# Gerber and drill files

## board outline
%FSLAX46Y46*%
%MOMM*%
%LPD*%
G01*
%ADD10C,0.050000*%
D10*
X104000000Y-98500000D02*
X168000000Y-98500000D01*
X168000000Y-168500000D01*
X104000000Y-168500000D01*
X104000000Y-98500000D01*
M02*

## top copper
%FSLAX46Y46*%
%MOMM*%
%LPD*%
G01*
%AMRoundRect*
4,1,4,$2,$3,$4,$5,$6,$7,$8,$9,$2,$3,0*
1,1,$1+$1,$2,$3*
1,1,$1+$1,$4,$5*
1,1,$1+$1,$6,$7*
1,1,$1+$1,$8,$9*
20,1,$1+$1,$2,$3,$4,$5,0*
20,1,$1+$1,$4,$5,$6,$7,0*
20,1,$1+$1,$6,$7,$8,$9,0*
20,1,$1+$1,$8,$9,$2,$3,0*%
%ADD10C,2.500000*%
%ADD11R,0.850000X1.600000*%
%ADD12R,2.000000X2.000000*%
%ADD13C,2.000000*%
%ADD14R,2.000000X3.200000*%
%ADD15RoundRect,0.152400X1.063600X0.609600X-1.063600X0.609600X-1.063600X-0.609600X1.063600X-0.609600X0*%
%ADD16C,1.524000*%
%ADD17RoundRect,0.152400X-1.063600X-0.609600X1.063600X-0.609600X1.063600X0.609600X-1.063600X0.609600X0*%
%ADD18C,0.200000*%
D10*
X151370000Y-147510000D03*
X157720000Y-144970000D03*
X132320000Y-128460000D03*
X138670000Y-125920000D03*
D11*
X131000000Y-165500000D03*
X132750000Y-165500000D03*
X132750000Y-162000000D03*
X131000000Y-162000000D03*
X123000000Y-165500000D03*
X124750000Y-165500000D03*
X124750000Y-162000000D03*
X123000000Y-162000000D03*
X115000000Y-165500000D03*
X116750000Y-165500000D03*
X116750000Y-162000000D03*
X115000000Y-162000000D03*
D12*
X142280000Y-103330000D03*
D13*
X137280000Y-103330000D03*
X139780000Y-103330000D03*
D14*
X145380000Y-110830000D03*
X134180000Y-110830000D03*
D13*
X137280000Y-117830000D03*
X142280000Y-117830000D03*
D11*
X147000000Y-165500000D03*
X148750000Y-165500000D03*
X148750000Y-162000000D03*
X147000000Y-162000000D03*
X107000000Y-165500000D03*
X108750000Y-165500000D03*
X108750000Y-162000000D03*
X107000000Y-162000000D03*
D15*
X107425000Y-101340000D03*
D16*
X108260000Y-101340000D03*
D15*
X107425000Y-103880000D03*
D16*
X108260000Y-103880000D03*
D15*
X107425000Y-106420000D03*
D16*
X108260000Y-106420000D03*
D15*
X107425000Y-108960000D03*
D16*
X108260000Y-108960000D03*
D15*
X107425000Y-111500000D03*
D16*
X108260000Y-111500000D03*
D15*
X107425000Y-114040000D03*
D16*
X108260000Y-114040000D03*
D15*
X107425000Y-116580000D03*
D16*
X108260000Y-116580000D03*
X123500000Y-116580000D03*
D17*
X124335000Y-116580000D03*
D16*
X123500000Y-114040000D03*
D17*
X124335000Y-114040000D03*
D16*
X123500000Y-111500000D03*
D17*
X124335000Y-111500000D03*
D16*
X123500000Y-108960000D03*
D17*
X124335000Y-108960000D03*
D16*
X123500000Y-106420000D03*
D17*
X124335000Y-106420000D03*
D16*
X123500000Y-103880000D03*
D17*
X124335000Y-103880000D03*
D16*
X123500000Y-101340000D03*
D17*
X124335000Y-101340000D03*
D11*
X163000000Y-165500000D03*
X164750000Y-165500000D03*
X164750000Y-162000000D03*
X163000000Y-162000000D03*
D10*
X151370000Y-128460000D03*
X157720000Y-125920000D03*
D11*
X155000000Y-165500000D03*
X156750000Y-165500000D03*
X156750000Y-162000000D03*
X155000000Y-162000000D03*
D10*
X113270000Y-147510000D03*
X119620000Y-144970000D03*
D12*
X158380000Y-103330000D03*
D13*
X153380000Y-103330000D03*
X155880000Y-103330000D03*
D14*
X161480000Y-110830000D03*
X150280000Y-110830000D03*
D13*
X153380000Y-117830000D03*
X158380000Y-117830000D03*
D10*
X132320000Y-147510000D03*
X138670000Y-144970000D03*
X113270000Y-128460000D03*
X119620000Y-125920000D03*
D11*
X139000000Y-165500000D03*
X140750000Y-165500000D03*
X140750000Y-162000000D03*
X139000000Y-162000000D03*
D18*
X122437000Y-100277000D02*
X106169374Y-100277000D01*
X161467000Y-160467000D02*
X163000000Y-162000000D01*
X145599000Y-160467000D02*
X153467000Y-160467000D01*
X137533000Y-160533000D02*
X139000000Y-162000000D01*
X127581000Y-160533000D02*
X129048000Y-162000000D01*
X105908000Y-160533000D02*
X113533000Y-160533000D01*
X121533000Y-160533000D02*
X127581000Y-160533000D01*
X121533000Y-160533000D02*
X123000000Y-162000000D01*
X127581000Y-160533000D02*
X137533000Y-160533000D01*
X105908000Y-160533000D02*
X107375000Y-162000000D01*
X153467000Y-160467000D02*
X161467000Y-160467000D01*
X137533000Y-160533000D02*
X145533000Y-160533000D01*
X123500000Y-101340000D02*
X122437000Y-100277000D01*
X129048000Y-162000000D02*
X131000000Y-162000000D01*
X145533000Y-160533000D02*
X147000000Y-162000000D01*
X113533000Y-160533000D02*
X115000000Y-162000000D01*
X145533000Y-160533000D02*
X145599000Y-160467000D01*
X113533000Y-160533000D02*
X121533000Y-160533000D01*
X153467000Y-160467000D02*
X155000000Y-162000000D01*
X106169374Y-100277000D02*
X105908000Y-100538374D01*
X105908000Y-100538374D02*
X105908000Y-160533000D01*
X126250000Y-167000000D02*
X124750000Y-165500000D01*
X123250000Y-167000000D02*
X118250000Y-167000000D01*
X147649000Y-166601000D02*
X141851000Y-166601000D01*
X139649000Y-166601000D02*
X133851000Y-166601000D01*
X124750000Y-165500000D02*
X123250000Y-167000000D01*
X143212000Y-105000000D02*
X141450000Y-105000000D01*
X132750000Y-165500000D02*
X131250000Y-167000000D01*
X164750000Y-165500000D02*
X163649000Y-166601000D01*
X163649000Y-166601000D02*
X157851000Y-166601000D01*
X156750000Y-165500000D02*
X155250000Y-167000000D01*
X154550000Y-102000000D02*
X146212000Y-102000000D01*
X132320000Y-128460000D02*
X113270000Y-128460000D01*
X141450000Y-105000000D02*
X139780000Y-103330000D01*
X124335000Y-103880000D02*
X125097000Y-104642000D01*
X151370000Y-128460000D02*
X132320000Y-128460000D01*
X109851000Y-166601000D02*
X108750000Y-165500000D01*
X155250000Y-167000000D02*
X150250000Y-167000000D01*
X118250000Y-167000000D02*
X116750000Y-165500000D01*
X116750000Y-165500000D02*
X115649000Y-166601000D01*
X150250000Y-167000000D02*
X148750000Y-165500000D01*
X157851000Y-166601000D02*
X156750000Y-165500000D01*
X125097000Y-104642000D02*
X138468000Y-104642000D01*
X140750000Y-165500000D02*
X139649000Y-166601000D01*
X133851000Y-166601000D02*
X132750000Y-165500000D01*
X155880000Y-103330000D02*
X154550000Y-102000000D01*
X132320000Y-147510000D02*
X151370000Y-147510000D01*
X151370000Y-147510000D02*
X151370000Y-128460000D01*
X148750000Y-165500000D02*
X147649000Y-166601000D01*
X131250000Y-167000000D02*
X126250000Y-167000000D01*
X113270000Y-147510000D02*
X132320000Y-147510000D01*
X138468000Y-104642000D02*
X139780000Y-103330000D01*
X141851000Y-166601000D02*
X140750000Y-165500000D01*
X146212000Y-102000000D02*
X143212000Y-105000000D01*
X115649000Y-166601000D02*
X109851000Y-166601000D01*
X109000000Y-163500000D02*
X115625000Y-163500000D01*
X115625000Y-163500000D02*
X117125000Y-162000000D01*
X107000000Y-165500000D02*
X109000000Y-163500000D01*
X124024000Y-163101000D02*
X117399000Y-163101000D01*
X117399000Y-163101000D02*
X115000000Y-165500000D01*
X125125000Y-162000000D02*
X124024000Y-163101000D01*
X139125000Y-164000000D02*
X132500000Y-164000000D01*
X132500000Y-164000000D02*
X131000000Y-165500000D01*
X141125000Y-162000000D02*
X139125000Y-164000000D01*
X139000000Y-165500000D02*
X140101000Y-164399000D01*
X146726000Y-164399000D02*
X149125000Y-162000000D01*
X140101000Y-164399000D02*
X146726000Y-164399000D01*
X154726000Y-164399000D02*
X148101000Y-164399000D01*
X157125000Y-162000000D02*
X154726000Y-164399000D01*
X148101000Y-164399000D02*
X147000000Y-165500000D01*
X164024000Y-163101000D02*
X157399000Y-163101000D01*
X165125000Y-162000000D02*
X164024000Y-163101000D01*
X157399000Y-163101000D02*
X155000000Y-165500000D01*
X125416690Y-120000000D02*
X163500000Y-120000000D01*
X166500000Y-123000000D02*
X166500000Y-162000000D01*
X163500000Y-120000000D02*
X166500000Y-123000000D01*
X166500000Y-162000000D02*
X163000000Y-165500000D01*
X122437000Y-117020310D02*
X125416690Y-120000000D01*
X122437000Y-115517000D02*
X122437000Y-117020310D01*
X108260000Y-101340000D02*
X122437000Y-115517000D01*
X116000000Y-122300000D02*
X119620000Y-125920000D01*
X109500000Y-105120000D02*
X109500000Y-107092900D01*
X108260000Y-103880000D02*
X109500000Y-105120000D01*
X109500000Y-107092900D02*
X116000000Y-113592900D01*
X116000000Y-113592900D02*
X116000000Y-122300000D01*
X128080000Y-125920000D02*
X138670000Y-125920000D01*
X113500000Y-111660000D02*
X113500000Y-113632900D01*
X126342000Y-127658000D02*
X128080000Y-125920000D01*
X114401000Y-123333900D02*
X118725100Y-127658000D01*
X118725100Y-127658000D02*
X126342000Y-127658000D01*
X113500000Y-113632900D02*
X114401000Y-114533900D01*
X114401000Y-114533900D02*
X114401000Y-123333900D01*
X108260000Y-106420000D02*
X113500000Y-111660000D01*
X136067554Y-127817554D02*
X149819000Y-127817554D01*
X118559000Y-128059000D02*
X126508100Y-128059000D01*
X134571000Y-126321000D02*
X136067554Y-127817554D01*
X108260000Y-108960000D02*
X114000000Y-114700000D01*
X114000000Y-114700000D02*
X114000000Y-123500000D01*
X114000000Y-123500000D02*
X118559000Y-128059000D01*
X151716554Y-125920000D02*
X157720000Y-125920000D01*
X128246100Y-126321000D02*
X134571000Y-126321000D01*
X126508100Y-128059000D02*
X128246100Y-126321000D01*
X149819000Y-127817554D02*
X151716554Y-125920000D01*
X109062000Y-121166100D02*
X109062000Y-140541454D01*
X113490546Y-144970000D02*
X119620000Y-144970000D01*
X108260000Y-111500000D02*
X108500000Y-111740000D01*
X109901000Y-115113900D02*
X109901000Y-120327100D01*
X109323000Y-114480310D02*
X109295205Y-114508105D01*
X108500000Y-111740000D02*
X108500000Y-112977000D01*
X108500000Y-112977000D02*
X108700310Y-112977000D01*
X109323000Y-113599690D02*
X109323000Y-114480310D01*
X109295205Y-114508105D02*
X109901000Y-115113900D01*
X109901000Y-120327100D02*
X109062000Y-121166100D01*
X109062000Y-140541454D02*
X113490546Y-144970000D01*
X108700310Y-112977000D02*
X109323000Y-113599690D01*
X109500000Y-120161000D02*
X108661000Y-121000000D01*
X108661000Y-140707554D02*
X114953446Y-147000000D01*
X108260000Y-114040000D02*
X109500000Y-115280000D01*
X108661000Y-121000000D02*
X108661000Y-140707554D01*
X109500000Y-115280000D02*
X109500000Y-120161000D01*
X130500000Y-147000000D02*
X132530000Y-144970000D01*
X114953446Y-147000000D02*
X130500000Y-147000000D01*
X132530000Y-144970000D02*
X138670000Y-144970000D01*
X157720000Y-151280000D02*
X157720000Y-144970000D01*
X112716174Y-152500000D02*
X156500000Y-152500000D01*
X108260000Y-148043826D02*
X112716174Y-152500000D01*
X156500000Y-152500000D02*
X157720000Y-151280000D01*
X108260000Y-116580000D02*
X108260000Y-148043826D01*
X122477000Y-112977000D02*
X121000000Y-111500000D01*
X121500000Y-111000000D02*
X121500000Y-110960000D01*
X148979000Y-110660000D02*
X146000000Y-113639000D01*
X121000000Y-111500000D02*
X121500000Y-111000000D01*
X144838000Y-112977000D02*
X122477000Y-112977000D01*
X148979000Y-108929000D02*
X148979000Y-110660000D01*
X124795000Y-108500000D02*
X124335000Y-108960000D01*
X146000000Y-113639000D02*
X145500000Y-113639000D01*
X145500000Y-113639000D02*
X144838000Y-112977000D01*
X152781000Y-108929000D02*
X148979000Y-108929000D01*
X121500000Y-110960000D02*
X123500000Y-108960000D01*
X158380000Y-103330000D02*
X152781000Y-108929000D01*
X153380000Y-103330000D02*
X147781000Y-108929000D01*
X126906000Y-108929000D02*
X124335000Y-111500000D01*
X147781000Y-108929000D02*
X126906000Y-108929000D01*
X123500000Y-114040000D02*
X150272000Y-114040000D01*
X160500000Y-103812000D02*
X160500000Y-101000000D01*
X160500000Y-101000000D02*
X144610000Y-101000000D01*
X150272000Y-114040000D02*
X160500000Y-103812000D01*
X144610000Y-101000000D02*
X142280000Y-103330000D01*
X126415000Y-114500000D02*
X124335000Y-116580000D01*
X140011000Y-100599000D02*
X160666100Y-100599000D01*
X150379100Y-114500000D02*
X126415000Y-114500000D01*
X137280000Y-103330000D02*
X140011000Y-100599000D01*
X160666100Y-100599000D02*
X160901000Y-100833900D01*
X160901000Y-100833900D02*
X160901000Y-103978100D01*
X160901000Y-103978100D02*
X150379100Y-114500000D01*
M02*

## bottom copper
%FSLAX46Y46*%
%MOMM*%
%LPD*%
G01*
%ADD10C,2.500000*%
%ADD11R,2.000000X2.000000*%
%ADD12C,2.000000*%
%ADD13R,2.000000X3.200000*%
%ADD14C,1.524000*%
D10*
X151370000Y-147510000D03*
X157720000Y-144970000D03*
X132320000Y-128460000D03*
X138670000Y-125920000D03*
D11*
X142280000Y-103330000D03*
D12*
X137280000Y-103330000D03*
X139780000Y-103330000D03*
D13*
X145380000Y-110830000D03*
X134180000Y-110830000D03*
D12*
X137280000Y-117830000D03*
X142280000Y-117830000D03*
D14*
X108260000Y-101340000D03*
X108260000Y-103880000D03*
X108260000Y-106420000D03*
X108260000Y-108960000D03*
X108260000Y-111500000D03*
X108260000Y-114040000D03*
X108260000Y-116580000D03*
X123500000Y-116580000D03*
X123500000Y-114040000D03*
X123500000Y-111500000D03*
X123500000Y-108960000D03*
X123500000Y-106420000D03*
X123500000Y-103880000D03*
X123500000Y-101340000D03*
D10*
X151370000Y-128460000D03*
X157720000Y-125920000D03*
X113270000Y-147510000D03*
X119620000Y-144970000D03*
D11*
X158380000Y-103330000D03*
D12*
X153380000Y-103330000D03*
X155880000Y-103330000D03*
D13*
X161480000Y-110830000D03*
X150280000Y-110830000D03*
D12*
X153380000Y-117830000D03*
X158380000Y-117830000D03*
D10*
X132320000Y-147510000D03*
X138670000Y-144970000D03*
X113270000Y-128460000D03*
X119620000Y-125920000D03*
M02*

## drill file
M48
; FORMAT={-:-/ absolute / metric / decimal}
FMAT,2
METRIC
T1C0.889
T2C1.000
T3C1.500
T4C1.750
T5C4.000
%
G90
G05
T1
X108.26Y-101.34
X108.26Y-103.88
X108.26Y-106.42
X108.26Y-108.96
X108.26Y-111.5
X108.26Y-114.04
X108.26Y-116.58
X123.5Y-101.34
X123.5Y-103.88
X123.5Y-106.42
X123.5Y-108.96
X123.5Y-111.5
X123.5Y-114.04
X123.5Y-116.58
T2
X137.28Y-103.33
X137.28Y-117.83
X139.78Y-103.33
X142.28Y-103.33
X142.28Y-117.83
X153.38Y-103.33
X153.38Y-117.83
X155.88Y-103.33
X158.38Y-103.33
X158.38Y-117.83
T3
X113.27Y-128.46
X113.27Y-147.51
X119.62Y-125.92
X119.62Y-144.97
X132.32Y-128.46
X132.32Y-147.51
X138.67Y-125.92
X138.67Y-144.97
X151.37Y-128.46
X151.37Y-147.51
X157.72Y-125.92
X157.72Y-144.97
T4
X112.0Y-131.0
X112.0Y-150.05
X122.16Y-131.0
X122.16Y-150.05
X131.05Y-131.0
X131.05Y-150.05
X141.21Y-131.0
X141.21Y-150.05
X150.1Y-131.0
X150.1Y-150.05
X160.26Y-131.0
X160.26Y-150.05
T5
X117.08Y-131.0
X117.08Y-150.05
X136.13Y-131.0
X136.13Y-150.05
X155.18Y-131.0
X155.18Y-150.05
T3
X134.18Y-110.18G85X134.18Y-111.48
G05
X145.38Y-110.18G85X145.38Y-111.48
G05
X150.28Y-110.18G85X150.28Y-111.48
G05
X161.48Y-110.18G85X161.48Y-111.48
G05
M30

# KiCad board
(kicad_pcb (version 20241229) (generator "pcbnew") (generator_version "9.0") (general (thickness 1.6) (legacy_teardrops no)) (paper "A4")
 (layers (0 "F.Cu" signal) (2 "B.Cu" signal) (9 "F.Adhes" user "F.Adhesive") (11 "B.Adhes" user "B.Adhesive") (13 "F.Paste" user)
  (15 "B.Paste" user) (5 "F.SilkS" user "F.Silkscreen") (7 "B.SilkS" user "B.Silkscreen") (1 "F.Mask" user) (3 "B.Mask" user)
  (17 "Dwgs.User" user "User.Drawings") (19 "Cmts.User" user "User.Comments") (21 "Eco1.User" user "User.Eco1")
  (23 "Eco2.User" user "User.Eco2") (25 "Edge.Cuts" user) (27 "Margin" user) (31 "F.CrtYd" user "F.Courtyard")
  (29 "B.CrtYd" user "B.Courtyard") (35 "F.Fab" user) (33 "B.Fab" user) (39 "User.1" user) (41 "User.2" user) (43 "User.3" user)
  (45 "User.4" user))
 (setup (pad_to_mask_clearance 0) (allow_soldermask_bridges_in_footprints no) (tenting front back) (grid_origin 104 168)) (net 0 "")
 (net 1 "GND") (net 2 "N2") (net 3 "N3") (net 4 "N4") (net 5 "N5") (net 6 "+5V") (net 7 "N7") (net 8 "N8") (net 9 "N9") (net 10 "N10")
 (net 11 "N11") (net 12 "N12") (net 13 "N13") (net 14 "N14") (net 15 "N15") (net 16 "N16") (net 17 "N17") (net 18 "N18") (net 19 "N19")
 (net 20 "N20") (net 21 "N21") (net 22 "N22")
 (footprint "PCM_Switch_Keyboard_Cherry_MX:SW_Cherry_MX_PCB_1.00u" (layer "F.Cu") (at 155.18 150.05)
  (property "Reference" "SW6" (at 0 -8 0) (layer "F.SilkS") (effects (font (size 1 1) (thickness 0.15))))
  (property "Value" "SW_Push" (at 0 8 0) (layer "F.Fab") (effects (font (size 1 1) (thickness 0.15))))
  (pad "" np_thru_hole circle (at -5.08 0) (size 1.75 1.75) (drill 1.75) (layers "*.Cu" "*.Mask"))
  (pad "" np_thru_hole circle (at 0 0) (size 4 4) (drill 4) (layers "*.Cu" "*.Mask"))
  (pad "" np_thru_hole circle (at 5.08 0) (size 1.75 1.75) (drill 1.75) (layers "*.Cu" "*.Mask"))
  (pad "1" thru_hole circle (at -3.81 -2.54) (size 2.5 2.5) (drill 1.5) (layers "*.Cu" "*.Mask") (remove_unused_layers no) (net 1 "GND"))
  (pad "2" thru_hole circle (at 2.54 -5.08) (size 2.5 2.5) (drill 1.5) (layers "*.Cu" "*.Mask") (remove_unused_layers no) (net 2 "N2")))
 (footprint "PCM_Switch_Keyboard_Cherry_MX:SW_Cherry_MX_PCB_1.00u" (layer "F.Cu") (at 136.13 131)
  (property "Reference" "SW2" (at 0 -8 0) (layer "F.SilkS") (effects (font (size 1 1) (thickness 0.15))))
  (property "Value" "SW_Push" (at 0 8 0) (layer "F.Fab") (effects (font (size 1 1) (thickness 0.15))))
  (pad "" np_thru_hole circle (at -5.08 0) (size 1.75 1.75) (drill 1.75) (layers "*.Cu" "*.Mask"))
  (pad "" np_thru_hole circle (at 0 0) (size 4 4) (drill 4) (layers "*.Cu" "*.Mask"))
  (pad "" np_thru_hole circle (at 5.08 0) (size 1.75 1.75) (drill 1.75) (layers "*.Cu" "*.Mask"))
  (pad "1" thru_hole circle (at -3.81 -2.54) (size 2.5 2.5) (drill 1.5) (layers "*.Cu" "*.Mask") (remove_unused_layers no) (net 1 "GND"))
  (pad "2" thru_hole circle (at 2.54 -5.08) (size 2.5 2.5) (drill 1.5) (layers "*.Cu" "*.Mask") (remove_unused_layers no) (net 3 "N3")))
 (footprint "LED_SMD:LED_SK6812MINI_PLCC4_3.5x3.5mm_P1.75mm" (layer "F.Cu") (at 131.875 163.75 90)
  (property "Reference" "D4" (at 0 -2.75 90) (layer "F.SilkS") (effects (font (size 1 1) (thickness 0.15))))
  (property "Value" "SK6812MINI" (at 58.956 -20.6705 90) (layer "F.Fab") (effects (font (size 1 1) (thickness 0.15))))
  (pad "1" smd rect (at -1.75 -0.875 90) (size 1.6 0.85) (layers "F.Cu" "F.Mask" "F.Paste") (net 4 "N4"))
  (pad "2" smd rect (at -1.75 0.875 90) (size 1.6 0.85) (layers "F.Cu" "F.Mask" "F.Paste") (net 1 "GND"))
  (pad "3" smd rect (at 1.75 0.875 90) (size 1.6 0.85) (layers "F.Cu" "F.Mask" "F.Paste") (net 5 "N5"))
  (pad "4" smd rect (at 1.75 -0.875 90) (size 1.6 0.85) (layers "F.Cu" "F.Mask" "F.Paste") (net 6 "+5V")))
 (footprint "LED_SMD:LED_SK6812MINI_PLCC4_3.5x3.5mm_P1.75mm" (layer "F.Cu") (at 123.875 163.75 90)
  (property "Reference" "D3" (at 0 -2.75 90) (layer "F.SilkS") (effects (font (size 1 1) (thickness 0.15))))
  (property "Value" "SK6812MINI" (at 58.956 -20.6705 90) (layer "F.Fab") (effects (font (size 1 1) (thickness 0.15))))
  (pad "1" smd rect (at -1.75 -0.875 90) (size 1.6 0.85) (layers "F.Cu" "F.Mask" "F.Paste") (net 5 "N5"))
  (pad "2" smd rect (at -1.75 0.875 90) (size 1.6 0.85) (layers "F.Cu" "F.Mask" "F.Paste") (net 1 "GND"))
  (pad "3" smd rect (at 1.75 0.875 90) (size 1.6 0.85) (layers "F.Cu" "F.Mask" "F.Paste") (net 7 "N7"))
  (pad "4" smd rect (at 1.75 -0.875 90) (size 1.6 0.85) (layers "F.Cu" "F.Mask" "F.Paste") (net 6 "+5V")))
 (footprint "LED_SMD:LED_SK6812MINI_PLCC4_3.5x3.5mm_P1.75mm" (layer "F.Cu") (at 115.875 163.75 90)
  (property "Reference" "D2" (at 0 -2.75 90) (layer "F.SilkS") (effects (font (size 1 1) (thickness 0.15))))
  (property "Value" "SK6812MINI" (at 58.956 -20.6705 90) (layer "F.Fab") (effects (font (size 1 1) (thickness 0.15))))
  (pad "1" smd rect (at -1.75 -0.875 90) (size 1.6 0.85) (layers "F.Cu" "F.Mask" "F.Paste") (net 7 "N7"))
  (pad "2" smd rect (at -1.75 0.875 90) (size 1.6 0.85) (layers "F.Cu" "F.Mask" "F.Paste") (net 1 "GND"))
  (pad "3" smd rect (at 1.75 0.875 90) (size 1.6 0.85) (layers "F.Cu" "F.Mask" "F.Paste") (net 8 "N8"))
  (pad "4" smd rect (at 1.75 -0.875 90) (size 1.6 0.85) (layers "F.Cu" "F.Mask" "F.Paste") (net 6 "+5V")))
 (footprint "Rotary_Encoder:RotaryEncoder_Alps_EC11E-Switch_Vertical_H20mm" (layer "F.Cu") (at 142.28 103.33 -90)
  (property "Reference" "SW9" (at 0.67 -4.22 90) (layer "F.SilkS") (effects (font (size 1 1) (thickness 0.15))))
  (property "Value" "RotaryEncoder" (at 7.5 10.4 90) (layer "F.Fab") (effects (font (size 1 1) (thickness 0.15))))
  (pad "A" thru_hole rect (at 0 0 270) (size 2 2) (drill 1) (layers "*.Cu" "*.Mask") (remove_unused_layers no) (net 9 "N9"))
  (pad "B" thru_hole circle (at 0 5 270) (size 2 2) (drill 1) (layers "*.Cu" "*.Mask") (remove_unused_layers no) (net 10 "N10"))
  (pad "C" thru_hole circle (at 0 2.5 270) (size 2 2) (drill 1) (layers "*.Cu" "*.Mask") (remove_unused_layers no) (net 1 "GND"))
  (pad "MP" thru_hole rect (at 7.5 -3.1 270) (size 3.2 2) (drill oval 2.8 1.5) (layers "*.Cu" "*.Mask") (remove_unused_layers no))
  (pad "MP" thru_hole rect (at 7.5 8.1 270) (size 3.2 2) (drill oval 2.8 1.5) (layers "*.Cu" "*.Mask") (remove_unused_layers no))
  (pad "S1" thru_hole circle (at 14.5 5 270) (size 2 2) (drill 1) (layers "*.Cu" "*.Mask") (remove_unused_layers no))
  (pad "S2" thru_hole circle (at 14.5 0 270) (size 2 2) (drill 1) (layers "*.Cu" "*.Mask") (remove_unused_layers no)))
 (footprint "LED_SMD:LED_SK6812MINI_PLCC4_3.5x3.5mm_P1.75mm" (layer "F.Cu") (at 147.875 163.75 90)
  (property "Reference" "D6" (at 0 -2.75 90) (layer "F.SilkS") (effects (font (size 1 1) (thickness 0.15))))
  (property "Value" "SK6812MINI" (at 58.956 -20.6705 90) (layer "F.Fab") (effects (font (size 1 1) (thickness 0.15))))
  (pad "1" smd rect (at -1.75 -0.875 90) (size 1.6 0.85) (layers "F.Cu" "F.Mask" "F.Paste") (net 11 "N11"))
  (pad "2" smd rect (at -1.75 0.875 90) (size 1.6 0.85) (layers "F.Cu" "F.Mask" "F.Paste") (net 1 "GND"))
  (pad "3" smd rect (at 1.75 0.875 90) (size 1.6 0.85) (layers "F.Cu" "F.Mask" "F.Paste") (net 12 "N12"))
  (pad "4" smd rect (at 1.75 -0.875 90) (size 1.6 0.85) (layers "F.Cu" "F.Mask" "F.Paste") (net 6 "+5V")))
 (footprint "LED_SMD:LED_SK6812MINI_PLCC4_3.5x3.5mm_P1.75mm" (layer "F.Cu") (at 107.875 163.75 90)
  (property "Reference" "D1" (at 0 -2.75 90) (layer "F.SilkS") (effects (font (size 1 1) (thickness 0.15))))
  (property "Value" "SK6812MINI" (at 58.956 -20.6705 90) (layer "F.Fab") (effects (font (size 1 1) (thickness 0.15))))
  (pad "1" smd rect (at -1.75 -0.875 90) (size 1.6 0.85) (layers "F.Cu" "F.Mask" "F.Paste") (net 8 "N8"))
  (pad "2" smd rect (at -1.75 0.875 90) (size 1.6 0.85) (layers "F.Cu" "F.Mask" "F.Paste") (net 1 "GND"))
  (pad "3" smd rect (at 1.75 0.875 90) (size 1.6 0.85) (layers "F.Cu" "F.Mask" "F.Paste") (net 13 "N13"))
  (pad "4" smd rect (at 1.75 -0.875 90) (size 1.6 0.85) (layers "F.Cu" "F.Mask" "F.Paste") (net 6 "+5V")))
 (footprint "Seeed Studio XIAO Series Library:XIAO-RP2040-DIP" (layer "F.Cu") (at 115.88 108.96)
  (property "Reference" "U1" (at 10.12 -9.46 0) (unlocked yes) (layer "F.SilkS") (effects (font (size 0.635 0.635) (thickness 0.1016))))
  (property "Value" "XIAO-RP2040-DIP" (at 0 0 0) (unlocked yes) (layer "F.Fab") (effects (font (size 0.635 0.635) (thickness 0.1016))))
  (pad "1" smd roundrect (at -8.455 -7.62 180) (size 2.432 1.524) (layers "F.Cu" "F.Mask") (roundrect_rratio 0.1) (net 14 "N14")
   (thermal_bridge_angle 45))
  (pad "1" thru_hole circle (at -7.62 -7.62 180) (size 1.524 1.524) (drill 0.889) (layers "*.Cu" "*.Mask") (remove_unused_layers no)
   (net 14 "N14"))
  (pad "2" smd roundrect (at -8.455 -5.08 180) (size 2.432 1.524) (layers "F.Cu" "F.Mask") (roundrect_rratio 0.1) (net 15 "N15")
   (thermal_bridge_angle 45))
  (pad "2" thru_hole circle (at -7.62 -5.08 180) (size 1.524 1.524) (drill 0.889) (layers "*.Cu" "*.Mask") (remove_unused_layers no)
   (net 15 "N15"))
  (pad "3" smd roundrect (at -8.455 -2.54 180) (size 2.432 1.524) (layers "F.Cu" "F.Mask") (roundrect_rratio 0.1) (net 3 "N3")
   (thermal_bridge_angle 45))
  (pad "3" thru_hole circle (at -7.62 -2.54 180) (size 1.524 1.524) (drill 0.889) (layers "*.Cu" "*.Mask") (remove_unused_layers no)
   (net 3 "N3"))
  (pad "4" smd roundrect (at -8.455 0 180) (size 2.432 1.524) (layers "F.Cu" "F.Mask") (roundrect_rratio 0.1) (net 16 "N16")
   (thermal_bridge_angle 45))
  (pad "4" thru_hole circle (at -7.62 0 180) (size 1.524 1.524) (drill 0.889) (layers "*.Cu" "*.Mask") (remove_unused_layers no)
   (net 16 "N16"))
  (pad "5" smd roundrect (at -8.455 2.54 180) (size 2.432 1.524) (layers "F.Cu" "F.Mask") (roundrect_rratio 0.1) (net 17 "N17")
   (thermal_bridge_angle 45))
  (pad "5" thru_hole circle (at -7.62 2.54 180) (size 1.524 1.524) (drill 0.889) (layers "*.Cu" "*.Mask") (remove_unused_layers no)
   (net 17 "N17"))
  (pad "6" smd roundrect (at -8.455 5.08 180) (size 2.432 1.524) (layers "F.Cu" "F.Mask") (roundrect_rratio 0.1) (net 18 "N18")
   (thermal_bridge_angle 45))
  (pad "6" thru_hole circle (at -7.62 5.08 180) (size 1.524 1.524) (drill 0.889) (layers "*.Cu" "*.Mask") (remove_unused_layers no)
   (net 18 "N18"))
  (pad "7" smd roundrect (at -8.455 7.62 180) (size 2.432 1.524) (layers "F.Cu" "F.Mask") (roundrect_rratio 0.1) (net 2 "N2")
   (thermal_bridge_angle 45))
  (pad "7" thru_hole circle (at -7.62 7.62 180) (size 1.524 1.524) (drill 0.889) (layers "*.Cu" "*.Mask") (remove_unused_layers no)
   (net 2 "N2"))
  (pad "8" thru_hole circle (at 7.62 7.62) (size 1.524 1.524) (drill 0.889) (layers "*.Cu" "*.Mask") (remove_unused_layers no)
   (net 10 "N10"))
  (pad "8" smd roundrect (at 8.455 7.62) (size 2.432 1.524) (layers "F.Cu" "F.Mask") (roundrect_rratio 0.1) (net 10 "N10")
   (thermal_bridge_angle 45))
  (pad "9" thru_hole circle (at 7.62 5.08) (size 1.524 1.524) (drill 0.889) (layers "*.Cu" "*.Mask") (remove_unused_layers no) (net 9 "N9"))
  (pad "9" smd roundrect (at 8.455 5.08) (size 2.432 1.524) (layers "F.Cu" "F.Mask") (roundrect_rratio 0.1) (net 9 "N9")
   (thermal_bridge_angle 45))
  (pad "10" thru_hole circle (at 7.62 2.54) (size 1.524 1.524) (drill 0.889) (layers "*.Cu" "*.Mask") (remove_unused_layers no)
   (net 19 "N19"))
  (pad "10" smd roundrect (at 8.455 2.54) (size 2.432 1.524) (layers "F.Cu" "F.Mask") (roundrect_rratio 0.1) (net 19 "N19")
   (thermal_bridge_angle 45))
  (pad "11" thru_hole circle (at 7.62 0) (size 1.524 1.524) (drill 0.889) (layers "*.Cu" "*.Mask") (remove_unused_layers no) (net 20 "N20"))
  (pad "11" smd roundrect (at 8.455 0) (size 2.432 1.524) (layers "F.Cu" "F.Mask") (roundrect_rratio 0.1) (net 20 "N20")
   (thermal_bridge_angle 45))
  (pad "12" thru_hole circle (at 7.62 -2.54) (size 1.524 1.524) (drill 0.889) (layers "*.Cu" "*.Mask") (remove_unused_layers no)
   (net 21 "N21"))
  (pad "12" smd roundrect (at 8.455 -2.54) (size 2.432 1.524) (layers "F.Cu" "F.Mask") (roundrect_rratio 0.1) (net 21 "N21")
   (thermal_bridge_angle 45))
  (pad "13" thru_hole circle (at 7.62 -5.08) (size 1.524 1.524) (drill 0.889) (layers "*.Cu" "*.Mask") (remove_unused_layers no)
   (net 1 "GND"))
  (pad "13" smd roundrect (at 8.455 -5.08) (size 2.432 1.524) (layers "F.Cu" "F.Mask") (roundrect_rratio 0.1) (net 1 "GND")
   (thermal_bridge_angle 45))
  (pad "14" thru_hole circle (at 7.62 -7.62) (size 1.524 1.524) (drill 0.889) (layers "*.Cu" "*.Mask") (remove_unused_layers no)
   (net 6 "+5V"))
  (pad "14" smd roundrect (at 8.455 -7.62) (size 2.432 1.524) (layers "F.Cu" "F.Mask") (roundrect_rratio 0.1) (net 6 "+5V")
   (thermal_bridge_angle 45)))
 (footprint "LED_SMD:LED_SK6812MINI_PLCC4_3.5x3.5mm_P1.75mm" (layer "F.Cu") (at 163.875 163.75 90)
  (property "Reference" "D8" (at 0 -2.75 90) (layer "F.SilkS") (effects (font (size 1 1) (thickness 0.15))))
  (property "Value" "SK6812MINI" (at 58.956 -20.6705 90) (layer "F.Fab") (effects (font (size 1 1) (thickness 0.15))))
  (pad "1" smd rect (at -1.75 -0.875 90) (size 1.6 0.85) (layers "F.Cu" "F.Mask" "F.Paste") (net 14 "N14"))
  (pad "2" smd rect (at -1.75 0.875 90) (size 1.6 0.85) (layers "F.Cu" "F.Mask" "F.Paste") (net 1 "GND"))
  (pad "3" smd rect (at 1.75 0.875 90) (size 1.6 0.85) (layers "F.Cu" "F.Mask" "F.Paste") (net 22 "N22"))
  (pad "4" smd rect (at 1.75 -0.875 90) (size 1.6 0.85) (layers "F.Cu" "F.Mask" "F.Paste") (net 6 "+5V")))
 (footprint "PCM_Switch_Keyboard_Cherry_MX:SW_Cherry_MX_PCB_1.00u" (layer "F.Cu") (at 155.18 131)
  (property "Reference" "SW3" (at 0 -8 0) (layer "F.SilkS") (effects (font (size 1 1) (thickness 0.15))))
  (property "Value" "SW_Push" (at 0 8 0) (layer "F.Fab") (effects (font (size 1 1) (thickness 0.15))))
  (pad "" np_thru_hole circle (at -5.08 0) (size 1.75 1.75) (drill 1.75) (layers "*.Cu" "*.Mask"))
  (pad "" np_thru_hole circle (at 0 0) (size 4 4) (drill 4) (layers "*.Cu" "*.Mask"))
  (pad "" np_thru_hole circle (at 5.08 0) (size 1.75 1.75) (drill 1.75) (layers "*.Cu" "*.Mask"))
  (pad "1" thru_hole circle (at -3.81 -2.54) (size 2.5 2.5) (drill 1.5) (layers "*.Cu" "*.Mask") (remove_unused_layers no) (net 1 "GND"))
  (pad "2" thru_hole circle (at 2.54 -5.08) (size 2.5 2.5) (drill 1.5) (layers "*.Cu" "*.Mask") (remove_unused_layers no) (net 16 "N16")))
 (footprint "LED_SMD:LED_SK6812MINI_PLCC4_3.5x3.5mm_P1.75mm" (layer "F.Cu") (at 155.875 163.75 90)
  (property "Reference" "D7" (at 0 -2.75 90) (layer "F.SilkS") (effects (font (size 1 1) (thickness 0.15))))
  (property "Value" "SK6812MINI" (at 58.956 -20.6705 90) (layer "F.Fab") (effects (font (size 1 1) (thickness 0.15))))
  (pad "1" smd rect (at -1.75 -0.875 90) (size 1.6 0.85) (layers "F.Cu" "F.Mask" "F.Paste") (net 22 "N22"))
  (pad "2" smd rect (at -1.75 0.875 90) (size 1.6 0.85) (layers "F.Cu" "F.Mask" "F.Paste") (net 1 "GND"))
  (pad "3" smd rect (at 1.75 0.875 90) (size 1.6 0.85) (layers "F.Cu" "F.Mask" "F.Paste") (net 11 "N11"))
  (pad "4" smd rect (at 1.75 -0.875 90) (size 1.6 0.85) (layers "F.Cu" "F.Mask" "F.Paste") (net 6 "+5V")))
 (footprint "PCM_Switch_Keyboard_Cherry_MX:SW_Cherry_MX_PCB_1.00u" (layer "F.Cu") (at 117.08 150.05)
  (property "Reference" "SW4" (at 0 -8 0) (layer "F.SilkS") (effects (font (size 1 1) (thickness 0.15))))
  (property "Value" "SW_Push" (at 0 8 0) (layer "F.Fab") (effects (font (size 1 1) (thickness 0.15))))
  (pad "" np_thru_hole circle (at -5.08 0) (size 1.75 1.75) (drill 1.75) (layers "*.Cu" "*.Mask"))
  (pad "" np_thru_hole circle (at 0 0) (size 4 4) (drill 4) (layers "*.Cu" "*.Mask"))
  (pad "" np_thru_hole circle (at 5.08 0) (size 1.75 1.75) (drill 1.75) (layers "*.Cu" "*.Mask"))
  (pad "1" thru_hole circle (at -3.81 -2.54) (size 2.5 2.5) (drill 1.5) (layers "*.Cu" "*.Mask") (remove_unused_layers no) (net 1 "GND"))
  (pad "2" thru_hole circle (at 2.54 -5.08) (size 2.5 2.5) (drill 1.5) (layers "*.Cu" "*.Mask") (remove_unused_layers no) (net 17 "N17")))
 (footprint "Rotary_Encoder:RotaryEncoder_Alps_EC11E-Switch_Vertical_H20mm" (layer "F.Cu") (at 158.38 103.33 -90)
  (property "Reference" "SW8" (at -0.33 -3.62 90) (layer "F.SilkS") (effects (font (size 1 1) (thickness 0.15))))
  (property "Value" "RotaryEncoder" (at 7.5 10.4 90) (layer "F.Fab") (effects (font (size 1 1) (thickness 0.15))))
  (pad "A" thru_hole rect (at 0 0 270) (size 2 2) (drill 1) (layers "*.Cu" "*.Mask") (remove_unused_layers no) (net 20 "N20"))
  (pad "B" thru_hole circle (at 0 5 270) (size 2 2) (drill 1) (layers "*.Cu" "*.Mask") (remove_unused_layers no) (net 19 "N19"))
  (pad "C" thru_hole circle (at 0 2.5 270) (size 2 2) (drill 1) (layers "*.Cu" "*.Mask") (remove_unused_layers no) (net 1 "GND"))
  (pad "MP" thru_hole rect (at 7.5 -3.1 270) (size 3.2 2) (drill oval 2.8 1.5) (layers "*.Cu" "*.Mask") (remove_unused_layers no))
  (pad "MP" thru_hole rect (at 7.5 8.1 270) (size 3.2 2) (drill oval 2.8 1.5) (layers "*.Cu" "*.Mask") (remove_unused_layers no))
  (pad "S1" thru_hole circle (at 14.5 5 270) (size 2 2) (drill 1) (layers "*.Cu" "*.Mask") (remove_unused_layers no))
  (pad "S2" thru_hole circle (at 14.5 0 270) (size 2 2) (drill 1) (layers "*.Cu" "*.Mask") (remove_unused_layers no)))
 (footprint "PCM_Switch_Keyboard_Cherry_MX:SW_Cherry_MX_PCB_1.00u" (layer "F.Cu") (at 136.13 150.05)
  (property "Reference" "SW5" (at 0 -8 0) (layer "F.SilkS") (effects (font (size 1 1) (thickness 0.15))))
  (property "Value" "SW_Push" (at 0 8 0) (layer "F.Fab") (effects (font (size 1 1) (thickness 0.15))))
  (pad "" np_thru_hole circle (at -5.08 0) (size 1.75 1.75) (drill 1.75) (layers "*.Cu" "*.Mask"))
  (pad "" np_thru_hole circle (at 0 0) (size 4 4) (drill 4) (layers "*.Cu" "*.Mask"))
  (pad "" np_thru_hole circle (at 5.08 0) (size 1.75 1.75) (drill 1.75) (layers "*.Cu" "*.Mask"))
  (pad "1" thru_hole circle (at -3.81 -2.54) (size 2.5 2.5) (drill 1.5) (layers "*.Cu" "*.Mask") (remove_unused_layers no) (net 1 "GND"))
  (pad "2" thru_hole circle (at 2.54 -5.08) (size 2.5 2.5) (drill 1.5) (layers "*.Cu" "*.Mask") (remove_unused_layers no) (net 18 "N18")))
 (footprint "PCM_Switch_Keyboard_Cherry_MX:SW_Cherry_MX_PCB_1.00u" (layer "F.Cu") (at 117.08 131)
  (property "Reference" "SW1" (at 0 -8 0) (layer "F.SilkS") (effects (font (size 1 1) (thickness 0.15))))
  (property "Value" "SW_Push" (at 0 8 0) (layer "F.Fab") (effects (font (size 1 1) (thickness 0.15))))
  (pad "" np_thru_hole circle (at -5.08 0) (size 1.75 1.75) (drill 1.75) (layers "*.Cu" "*.Mask"))
  (pad "" np_thru_hole circle (at 0 0) (size 4 4) (drill 4) (layers "*.Cu" "*.Mask"))
  (pad "" np_thru_hole circle (at 5.08 0) (size 1.75 1.75) (drill 1.75) (layers "*.Cu" "*.Mask"))
  (pad "1" thru_hole circle (at -3.81 -2.54) (size 2.5 2.5) (drill 1.5) (layers "*.Cu" "*.Mask") (remove_unused_layers no) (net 1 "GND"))
  (pad "2" thru_hole circle (at 2.54 -5.08) (size 2.5 2.5) (drill 1.5) (layers "*.Cu" "*.Mask") (remove_unused_layers no) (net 15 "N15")))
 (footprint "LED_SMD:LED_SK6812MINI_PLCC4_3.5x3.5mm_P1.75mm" (layer "F.Cu") (at 139.875 163.75 90)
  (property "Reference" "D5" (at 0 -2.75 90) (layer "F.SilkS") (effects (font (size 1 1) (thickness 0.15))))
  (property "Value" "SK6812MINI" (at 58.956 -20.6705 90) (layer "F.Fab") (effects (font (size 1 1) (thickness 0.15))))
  (pad "1" smd rect (at -1.75 -0.875 90) (size 1.6 0.85) (layers "F.Cu" "F.Mask" "F.Paste") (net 12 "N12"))
  (pad "2" smd rect (at -1.75 0.875 90) (size 1.6 0.85) (layers "F.Cu" "F.Mask" "F.Paste") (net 1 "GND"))
  (pad "3" smd rect (at 1.75 0.875 90) (size 1.6 0.85) (layers "F.Cu" "F.Mask" "F.Paste") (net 4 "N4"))
  (pad "4" smd rect (at 1.75 -0.875 90) (size 1.6 0.85) (layers "F.Cu" "F.Mask" "F.Paste") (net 6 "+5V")))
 (gr_rect (start 104 98.5) (end 168 168.5) (stroke (width 0.05) (type default)) (fill no) (layer "Edge.Cuts"))
 (segment (start 122.437 100.277) (end 106.169374 100.277) (width 0.2) (layer "F.Cu") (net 6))
 (segment (start 161.467 160.467) (end 163 162) (width 0.2) (layer "F.Cu") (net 6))
 (segment (start 145.599 160.467) (end 153.467 160.467) (width 0.2) (layer "F.Cu") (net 6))
 (segment (start 137.533 160.533) (end 139 162) (width 0.2) (layer "F.Cu") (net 6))
 (segment (start 127.581 160.533) (end 129.048 162) (width 0.2) (layer "F.Cu") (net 6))
 (segment (start 105.908 160.533) (end 113.533 160.533) (width 0.2) (layer "F.Cu") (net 6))
 (segment (start 121.533 160.533) (end 127.581 160.533) (width 0.2) (layer "F.Cu") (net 6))
 (segment (start 121.533 160.533) (end 123 162) (width 0.2) (layer "F.Cu") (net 6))
 (segment (start 127.581 160.533) (end 137.533 160.533) (width 0.2) (layer "F.Cu") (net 6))
 (segment (start 105.908 160.533) (end 107.375 162) (width 0.2) (layer "F.Cu") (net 6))
 (segment (start 153.467 160.467) (end 161.467 160.467) (width 0.2) (layer "F.Cu") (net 6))
 (segment (start 137.533 160.533) (end 145.533 160.533) (width 0.2) (layer "F.Cu") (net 6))
 (segment (start 123.5 101.34) (end 122.437 100.277) (width 0.2) (layer "F.Cu") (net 6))
 (segment (start 129.048 162) (end 131 162) (width 0.2) (layer "F.Cu") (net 6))
 (segment (start 145.533 160.533) (end 147 162) (width 0.2) (layer "F.Cu") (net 6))
 (segment (start 113.533 160.533) (end 115 162) (width 0.2) (layer "F.Cu") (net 6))
 (segment (start 145.533 160.533) (end 145.599 160.467) (width 0.2) (layer "F.Cu") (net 6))
 (segment (start 113.533 160.533) (end 121.533 160.533) (width 0.2) (layer "F.Cu") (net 6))
 (segment (start 153.467 160.467) (end 155 162) (width 0.2) (layer "F.Cu") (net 6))
 (segment (start 106.169374 100.277) (end 105.908 100.538374) (width 0.2) (layer "F.Cu") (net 6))
 (segment (start 105.908 100.538374) (end 105.908 160.533) (width 0.2) (layer "F.Cu") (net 6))
 (segment (start 126.25 167) (end 124.75 165.5) (width 0.2) (layer "F.Cu") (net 1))
 (segment (start 123.25 167) (end 118.25 167) (width 0.2) (layer "F.Cu") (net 1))
 (segment (start 147.649 166.601) (end 141.851 166.601) (width 0.2) (layer "F.Cu") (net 1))
 (segment (start 139.649 166.601) (end 133.851 166.601) (width 0.2) (layer "F.Cu") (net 1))
 (segment (start 124.75 165.5) (end 123.25 167) (width 0.2) (layer "F.Cu") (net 1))
 (segment (start 143.212 105) (end 141.45 105) (width 0.2) (layer "F.Cu") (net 1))
 (segment (start 132.75 165.5) (end 131.25 167) (width 0.2) (layer "F.Cu") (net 1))
 (segment (start 164.75 165.5) (end 163.649 166.601) (width 0.2) (layer "F.Cu") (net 1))
 (segment (start 163.649 166.601) (end 157.851 166.601) (width 0.2) (layer "F.Cu") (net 1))
 (segment (start 156.75 165.5) (end 155.25 167) (width 0.2) (layer "F.Cu") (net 1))
 (segment (start 154.55 102) (end 146.212 102) (width 0.2) (layer "F.Cu") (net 1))
 (segment (start 132.32 128.46) (end 113.27 128.46) (width 0.2) (layer "F.Cu") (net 1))
 (segment (start 141.45 105) (end 139.78 103.33) (width 0.2) (layer "F.Cu") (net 1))
 (segment (start 124.335 103.88) (end 125.097 104.642) (width 0.2) (layer "F.Cu") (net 1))
 (segment (start 151.37 128.46) (end 132.32 128.46) (width 0.2) (layer "F.Cu") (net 1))
 (segment (start 109.851 166.601) (end 108.75 165.5) (width 0.2) (layer "F.Cu") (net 1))
 (segment (start 155.25 167) (end 150.25 167) (width 0.2) (layer "F.Cu") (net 1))
 (segment (start 118.25 167) (end 116.75 165.5) (width 0.2) (layer "F.Cu") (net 1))
 (segment (start 116.75 165.5) (end 115.649 166.601) (width 0.2) (layer "F.Cu") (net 1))
 (segment (start 150.25 167) (end 148.75 165.5) (width 0.2) (layer "F.Cu") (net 1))
 (segment (start 157.851 166.601) (end 156.75 165.5) (width 0.2) (layer "F.Cu") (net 1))
 (segment (start 125.097 104.642) (end 138.468 104.642) (width 0.2) (layer "F.Cu") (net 1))
 (segment (start 140.75 165.5) (end 139.649 166.601) (width 0.2) (layer "F.Cu") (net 1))
 (segment (start 133.851 166.601) (end 132.75 165.5) (width 0.2) (layer "F.Cu") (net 1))
 (segment (start 155.88 103.33) (end 154.55 102) (width 0.2) (layer "F.Cu") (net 1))
 (segment (start 132.32 147.51) (end 151.37 147.51) (width 0.2) (layer "F.Cu") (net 1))
 (segment (start 151.37 147.51) (end 151.37 128.46) (width 0.2) (layer "F.Cu") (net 1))
 (segment (start 148.75 165.5) (end 147.649 166.601) (width 0.2) (layer "F.Cu") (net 1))
 (segment (start 131.25 167) (end 126.25 167) (width 0.2) (layer "F.Cu") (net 1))
 (segment (start 113.27 147.51) (end 132.32 147.51) (width 0.2) (layer "F.Cu") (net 1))
 (segment (start 138.468 104.642) (end 139.78 103.33) (width 0.2) (layer "F.Cu") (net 1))
 (segment (start 141.851 166.601) (end 140.75 165.5) (width 0.2) (layer "F.Cu") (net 1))
 (segment (start 146.212 102) (end 143.212 105) (width 0.2) (layer "F.Cu") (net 1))
 (segment (start 115.649 166.601) (end 109.851 166.601) (width 0.2) (layer "F.Cu") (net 1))
 (segment (start 109 163.5) (end 115.625 163.5) (width 0.2) (layer "F.Cu") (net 8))
 (segment (start 115.625 163.5) (end 117.125 162) (width 0.2) (layer "F.Cu") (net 8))
 (segment (start 107 165.5) (end 109 163.5) (width 0.2) (layer "F.Cu") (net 8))
 (segment (start 124.024 163.101) (end 117.399 163.101) (width 0.2) (layer "F.Cu") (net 7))
 (segment (start 117.399 163.101) (end 115 165.5) (width 0.2) (layer "F.Cu") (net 7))
 (segment (start 125.125 162) (end 124.024 163.101) (width 0.2) (layer "F.Cu") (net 7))
 (segment (start 139.125 164) (end 132.5 164) (width 0.2) (layer "F.Cu") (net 4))
 (segment (start 132.5 164) (end 131 165.5) (width 0.2) (layer "F.Cu") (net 4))
 (segment (start 141.125 162) (end 139.125 164) (width 0.2) (layer "F.Cu") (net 4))
 (segment (start 139 165.5) (end 140.101 164.399) (width 0.2) (layer "F.Cu") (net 12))
 (segment (start 146.726 164.399) (end 149.125 162) (width 0.2) (layer "F.Cu") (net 12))
 (segment (start 140.101 164.399) (end 146.726 164.399) (width 0.2) (layer "F.Cu") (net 12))
 (segment (start 154.726 164.399) (end 148.101 164.399) (width 0.2) (layer "F.Cu") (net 11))
 (segment (start 157.125 162) (end 154.726 164.399) (width 0.2) (layer "F.Cu") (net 11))
 (segment (start 148.101 164.399) (end 147 165.5) (width 0.2) (layer "F.Cu") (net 11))
 (segment (start 164.024 163.101) (end 157.399 163.101) (width 0.2) (layer "F.Cu") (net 22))
 (segment (start 165.125 162) (end 164.024 163.101) (width 0.2) (layer "F.Cu") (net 22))
 (segment (start 157.399 163.101) (end 155 165.5) (width 0.2) (layer "F.Cu") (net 22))
 (segment (start 125.41669 120) (end 163.5 120) (width 0.2) (layer "F.Cu") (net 14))
 (segment (start 166.5 123) (end 166.5 162) (width 0.2) (layer "F.Cu") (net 14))
 (segment (start 163.5 120) (end 166.5 123) (width 0.2) (layer "F.Cu") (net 14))
 (segment (start 166.5 162) (end 163 165.5) (width 0.2) (layer "F.Cu") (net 14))
 (segment (start 122.437 117.02031) (end 125.41669 120) (width 0.2) (layer "F.Cu") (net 14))
 (segment (start 122.437 115.517) (end 122.437 117.02031) (width 0.2) (layer "F.Cu") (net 14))
 (segment (start 108.26 101.34) (end 122.437 115.517) (width 0.2) (layer "F.Cu") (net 14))
 (segment (start 116 122.3) (end 119.62 125.92) (width 0.2) (layer "F.Cu") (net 15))
 (segment (start 109.5 105.12) (end 109.5 107.0929) (width 0.2) (layer "F.Cu") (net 15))
 (segment (start 108.26 103.88) (end 109.5 105.12) (width 0.2) (layer "F.Cu") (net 15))
 (segment (start 109.5 107.0929) (end 116 113.5929) (width 0.2) (layer "F.Cu") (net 15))
 (segment (start 116 113.5929) (end 116 122.3) (width 0.2) (layer "F.Cu") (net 15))
 (segment (start 128.08 125.92) (end 138.67 125.92) (width 0.2) (layer "F.Cu") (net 3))
 (segment (start 113.5 111.66) (end 113.5 113.6329) (width 0.2) (layer "F.Cu") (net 3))
 (segment (start 126.342 127.658) (end 128.08 125.92) (width 0.2) (layer "F.Cu") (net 3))
 (segment (start 114.401 123.3339) (end 118.7251 127.658) (width 0.2) (layer "F.Cu") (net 3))
 (segment (start 118.7251 127.658) (end 126.342 127.658) (width 0.2) (layer "F.Cu") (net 3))
 (segment (start 113.5 113.6329) (end 114.401 114.5339) (width 0.2) (layer "F.Cu") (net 3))
 (segment (start 114.401 114.5339) (end 114.401 123.3339) (width 0.2) (layer "F.Cu") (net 3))
 (segment (start 108.26 106.42) (end 113.5 111.66) (width 0.2) (layer "F.Cu") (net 3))
 (segment (start 136.067554 127.817554) (end 149.819 127.817554) (width 0.2) (layer "F.Cu") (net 16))
 (segment (start 118.559 128.059) (end 126.5081 128.059) (width 0.2) (layer "F.Cu") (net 16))
 (segment (start 134.571 126.321) (end 136.067554 127.817554) (width 0.2) (layer "F.Cu") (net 16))
 (segment (start 108.26 108.96) (end 114 114.7) (width 0.2) (layer "F.Cu") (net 16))
 (segment (start 114 114.7) (end 114 123.5) (width 0.2) (layer "F.Cu") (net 16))
 (segment (start 114 123.5) (end 118.559 128.059) (width 0.2) (layer "F.Cu") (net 16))
 (segment (start 151.716554 125.92) (end 157.72 125.92) (width 0.2) (layer "F.Cu") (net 16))
 (segment (start 128.2461 126.321) (end 134.571 126.321) (width 0.2) (layer "F.Cu") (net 16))
 (segment (start 126.5081 128.059) (end 128.2461 126.321) (width 0.2) (layer "F.Cu") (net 16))
 (segment (start 149.819 127.817554) (end 151.716554 125.92) (width 0.2) (layer "F.Cu") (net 16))
 (segment (start 109.062 121.1661) (end 109.062 140.541454) (width 0.2) (layer "F.Cu") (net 17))
 (segment (start 113.490546 144.97) (end 119.62 144.97) (width 0.2) (layer "F.Cu") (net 17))
 (segment (start 108.26 111.5) (end 108.5 111.74) (width 0.2) (layer "F.Cu") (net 17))
 (segment (start 109.901 115.1139) (end 109.901 120.3271) (width 0.2) (layer "F.Cu") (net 17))
 (segment (start 109.323 114.48031) (end 109.295205 114.508105) (width 0.2) (layer "F.Cu") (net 17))
 (segment (start 108.5 111.74) (end 108.5 112.977) (width 0.2) (layer "F.Cu") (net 17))
 (segment (start 108.5 112.977) (end 108.70031 112.977) (width 0.2) (layer "F.Cu") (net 17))
 (segment (start 109.323 113.59969) (end 109.323 114.48031) (width 0.2) (layer "F.Cu") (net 17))
 (segment (start 109.295205 114.508105) (end 109.901 115.1139) (width 0.2) (layer "F.Cu") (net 17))
 (segment (start 109.901 120.3271) (end 109.062 121.1661) (width 0.2) (layer "F.Cu") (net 17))
 (segment (start 109.062 140.541454) (end 113.490546 144.97) (width 0.2) (layer "F.Cu") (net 17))
 (segment (start 108.70031 112.977) (end 109.323 113.59969) (width 0.2) (layer "F.Cu") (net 17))
 (segment (start 109.5 120.161) (end 108.661 121) (width 0.2) (layer "F.Cu") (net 18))
 (segment (start 108.661 140.707554) (end 114.953446 147) (width 0.2) (layer "F.Cu") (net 18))
 (segment (start 108.26 114.04) (end 109.5 115.28) (width 0.2) (layer "F.Cu") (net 18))
 (segment (start 108.661 121) (end 108.661 140.707554) (width 0.2) (layer "F.Cu") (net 18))
 (segment (start 109.5 115.28) (end 109.5 120.161) (width 0.2) (layer "F.Cu") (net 18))
 (segment (start 130.5 147) (end 132.53 144.97) (width 0.2) (layer "F.Cu") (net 18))
 (segment (start 114.953446 147) (end 130.5 147) (width 0.2) (layer "F.Cu") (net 18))
 (segment (start 132.53 144.97) (end 138.67 144.97) (width 0.2) (layer "F.Cu") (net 18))
 (segment (start 157.72 151.28) (end 157.72 144.97) (width 0.2) (layer "F.Cu") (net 2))
 (segment (start 112.716174 152.5) (end 156.5 152.5) (width 0.2) (layer "F.Cu") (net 2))
 (segment (start 108.26 148.043826) (end 112.716174 152.5) (width 0.2) (layer "F.Cu") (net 2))
 (segment (start 156.5 152.5) (end 157.72 151.28) (width 0.2) (layer "F.Cu") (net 2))
 (segment (start 108.26 116.58) (end 108.26 148.043826) (width 0.2) (layer "F.Cu") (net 2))
 (segment (start 122.477 112.977) (end 121 111.5) (width 0.2) (layer "F.Cu") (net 20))
 (segment (start 121.5 111) (end 121.5 110.96) (width 0.2) (layer "F.Cu") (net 20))
 (segment (start 148.979 110.66) (end 146 113.639) (width 0.2) (layer "F.Cu") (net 20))
 (segment (start 121 111.5) (end 121.5 111) (width 0.2) (layer "F.Cu") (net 20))
 (segment (start 144.838 112.977) (end 122.477 112.977) (width 0.2) (layer "F.Cu") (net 20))
 (segment (start 148.979 108.929) (end 148.979 110.66) (width 0.2) (layer "F.Cu") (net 20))
 (segment (start 124.795 108.5) (end 124.335 108.96) (width 0.2) (layer "F.Cu") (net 20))
 (segment (start 146 113.639) (end 145.5 113.639) (width 0.2) (layer "F.Cu") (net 20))
 (segment (start 145.5 113.639) (end 144.838 112.977) (width 0.2) (layer "F.Cu") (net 20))
 (segment (start 152.781 108.929) (end 148.979 108.929) (width 0.2) (layer "F.Cu") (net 20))
 (segment (start 121.5 110.96) (end 123.5 108.96) (width 0.2) (layer "F.Cu") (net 20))
 (segment (start 158.38 103.33) (end 152.781 108.929) (width 0.2) (layer "F.Cu") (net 20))
 (segment (start 153.38 103.33) (end 147.781 108.929) (width 0.2) (layer "F.Cu") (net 19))
 (segment (start 126.906 108.929) (end 124.335 111.5) (width 0.2) (layer "F.Cu") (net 19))
 (segment (start 147.781 108.929) (end 126.906 108.929) (width 0.2) (layer "F.Cu") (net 19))
 (segment (start 123.5 114.04) (end 150.272 114.04) (width 0.2) (layer "F.Cu") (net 9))
 (segment (start 160.5 103.812) (end 160.5 101) (width 0.2) (layer "F.Cu") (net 9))
 (segment (start 160.5 101) (end 144.61 101) (width 0.2) (layer "F.Cu") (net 9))
 (segment (start 150.272 114.04) (end 160.5 103.812) (width 0.2) (layer "F.Cu") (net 9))
 (segment (start 144.61 101) (end 142.28 103.33) (width 0.2) (layer "F.Cu") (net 9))
 (segment (start 126.415 114.5) (end 124.335 116.58) (width 0.2) (layer "F.Cu") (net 10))
 (segment (start 140.011 100.599) (end 160.6661 100.599) (width 0.2) (layer "F.Cu") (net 10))
 (segment (start 150.3791 114.5) (end 126.415 114.5) (width 0.2) (layer "F.Cu") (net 10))
 (segment (start 137.28 103.33) (end 140.011 100.599) (width 0.2) (layer "F.Cu") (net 10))
 (segment (start 160.6661 100.599) (end 160.901 100.8339) (width 0.2) (layer "F.Cu") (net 10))
 (segment (start 160.901 100.8339) (end 160.901 103.9781) (width 0.2) (layer "F.Cu") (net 10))
 (segment (start 160.901 103.9781) (end 150.3791 114.5) (width 0.2) (layer "F.Cu") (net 10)))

